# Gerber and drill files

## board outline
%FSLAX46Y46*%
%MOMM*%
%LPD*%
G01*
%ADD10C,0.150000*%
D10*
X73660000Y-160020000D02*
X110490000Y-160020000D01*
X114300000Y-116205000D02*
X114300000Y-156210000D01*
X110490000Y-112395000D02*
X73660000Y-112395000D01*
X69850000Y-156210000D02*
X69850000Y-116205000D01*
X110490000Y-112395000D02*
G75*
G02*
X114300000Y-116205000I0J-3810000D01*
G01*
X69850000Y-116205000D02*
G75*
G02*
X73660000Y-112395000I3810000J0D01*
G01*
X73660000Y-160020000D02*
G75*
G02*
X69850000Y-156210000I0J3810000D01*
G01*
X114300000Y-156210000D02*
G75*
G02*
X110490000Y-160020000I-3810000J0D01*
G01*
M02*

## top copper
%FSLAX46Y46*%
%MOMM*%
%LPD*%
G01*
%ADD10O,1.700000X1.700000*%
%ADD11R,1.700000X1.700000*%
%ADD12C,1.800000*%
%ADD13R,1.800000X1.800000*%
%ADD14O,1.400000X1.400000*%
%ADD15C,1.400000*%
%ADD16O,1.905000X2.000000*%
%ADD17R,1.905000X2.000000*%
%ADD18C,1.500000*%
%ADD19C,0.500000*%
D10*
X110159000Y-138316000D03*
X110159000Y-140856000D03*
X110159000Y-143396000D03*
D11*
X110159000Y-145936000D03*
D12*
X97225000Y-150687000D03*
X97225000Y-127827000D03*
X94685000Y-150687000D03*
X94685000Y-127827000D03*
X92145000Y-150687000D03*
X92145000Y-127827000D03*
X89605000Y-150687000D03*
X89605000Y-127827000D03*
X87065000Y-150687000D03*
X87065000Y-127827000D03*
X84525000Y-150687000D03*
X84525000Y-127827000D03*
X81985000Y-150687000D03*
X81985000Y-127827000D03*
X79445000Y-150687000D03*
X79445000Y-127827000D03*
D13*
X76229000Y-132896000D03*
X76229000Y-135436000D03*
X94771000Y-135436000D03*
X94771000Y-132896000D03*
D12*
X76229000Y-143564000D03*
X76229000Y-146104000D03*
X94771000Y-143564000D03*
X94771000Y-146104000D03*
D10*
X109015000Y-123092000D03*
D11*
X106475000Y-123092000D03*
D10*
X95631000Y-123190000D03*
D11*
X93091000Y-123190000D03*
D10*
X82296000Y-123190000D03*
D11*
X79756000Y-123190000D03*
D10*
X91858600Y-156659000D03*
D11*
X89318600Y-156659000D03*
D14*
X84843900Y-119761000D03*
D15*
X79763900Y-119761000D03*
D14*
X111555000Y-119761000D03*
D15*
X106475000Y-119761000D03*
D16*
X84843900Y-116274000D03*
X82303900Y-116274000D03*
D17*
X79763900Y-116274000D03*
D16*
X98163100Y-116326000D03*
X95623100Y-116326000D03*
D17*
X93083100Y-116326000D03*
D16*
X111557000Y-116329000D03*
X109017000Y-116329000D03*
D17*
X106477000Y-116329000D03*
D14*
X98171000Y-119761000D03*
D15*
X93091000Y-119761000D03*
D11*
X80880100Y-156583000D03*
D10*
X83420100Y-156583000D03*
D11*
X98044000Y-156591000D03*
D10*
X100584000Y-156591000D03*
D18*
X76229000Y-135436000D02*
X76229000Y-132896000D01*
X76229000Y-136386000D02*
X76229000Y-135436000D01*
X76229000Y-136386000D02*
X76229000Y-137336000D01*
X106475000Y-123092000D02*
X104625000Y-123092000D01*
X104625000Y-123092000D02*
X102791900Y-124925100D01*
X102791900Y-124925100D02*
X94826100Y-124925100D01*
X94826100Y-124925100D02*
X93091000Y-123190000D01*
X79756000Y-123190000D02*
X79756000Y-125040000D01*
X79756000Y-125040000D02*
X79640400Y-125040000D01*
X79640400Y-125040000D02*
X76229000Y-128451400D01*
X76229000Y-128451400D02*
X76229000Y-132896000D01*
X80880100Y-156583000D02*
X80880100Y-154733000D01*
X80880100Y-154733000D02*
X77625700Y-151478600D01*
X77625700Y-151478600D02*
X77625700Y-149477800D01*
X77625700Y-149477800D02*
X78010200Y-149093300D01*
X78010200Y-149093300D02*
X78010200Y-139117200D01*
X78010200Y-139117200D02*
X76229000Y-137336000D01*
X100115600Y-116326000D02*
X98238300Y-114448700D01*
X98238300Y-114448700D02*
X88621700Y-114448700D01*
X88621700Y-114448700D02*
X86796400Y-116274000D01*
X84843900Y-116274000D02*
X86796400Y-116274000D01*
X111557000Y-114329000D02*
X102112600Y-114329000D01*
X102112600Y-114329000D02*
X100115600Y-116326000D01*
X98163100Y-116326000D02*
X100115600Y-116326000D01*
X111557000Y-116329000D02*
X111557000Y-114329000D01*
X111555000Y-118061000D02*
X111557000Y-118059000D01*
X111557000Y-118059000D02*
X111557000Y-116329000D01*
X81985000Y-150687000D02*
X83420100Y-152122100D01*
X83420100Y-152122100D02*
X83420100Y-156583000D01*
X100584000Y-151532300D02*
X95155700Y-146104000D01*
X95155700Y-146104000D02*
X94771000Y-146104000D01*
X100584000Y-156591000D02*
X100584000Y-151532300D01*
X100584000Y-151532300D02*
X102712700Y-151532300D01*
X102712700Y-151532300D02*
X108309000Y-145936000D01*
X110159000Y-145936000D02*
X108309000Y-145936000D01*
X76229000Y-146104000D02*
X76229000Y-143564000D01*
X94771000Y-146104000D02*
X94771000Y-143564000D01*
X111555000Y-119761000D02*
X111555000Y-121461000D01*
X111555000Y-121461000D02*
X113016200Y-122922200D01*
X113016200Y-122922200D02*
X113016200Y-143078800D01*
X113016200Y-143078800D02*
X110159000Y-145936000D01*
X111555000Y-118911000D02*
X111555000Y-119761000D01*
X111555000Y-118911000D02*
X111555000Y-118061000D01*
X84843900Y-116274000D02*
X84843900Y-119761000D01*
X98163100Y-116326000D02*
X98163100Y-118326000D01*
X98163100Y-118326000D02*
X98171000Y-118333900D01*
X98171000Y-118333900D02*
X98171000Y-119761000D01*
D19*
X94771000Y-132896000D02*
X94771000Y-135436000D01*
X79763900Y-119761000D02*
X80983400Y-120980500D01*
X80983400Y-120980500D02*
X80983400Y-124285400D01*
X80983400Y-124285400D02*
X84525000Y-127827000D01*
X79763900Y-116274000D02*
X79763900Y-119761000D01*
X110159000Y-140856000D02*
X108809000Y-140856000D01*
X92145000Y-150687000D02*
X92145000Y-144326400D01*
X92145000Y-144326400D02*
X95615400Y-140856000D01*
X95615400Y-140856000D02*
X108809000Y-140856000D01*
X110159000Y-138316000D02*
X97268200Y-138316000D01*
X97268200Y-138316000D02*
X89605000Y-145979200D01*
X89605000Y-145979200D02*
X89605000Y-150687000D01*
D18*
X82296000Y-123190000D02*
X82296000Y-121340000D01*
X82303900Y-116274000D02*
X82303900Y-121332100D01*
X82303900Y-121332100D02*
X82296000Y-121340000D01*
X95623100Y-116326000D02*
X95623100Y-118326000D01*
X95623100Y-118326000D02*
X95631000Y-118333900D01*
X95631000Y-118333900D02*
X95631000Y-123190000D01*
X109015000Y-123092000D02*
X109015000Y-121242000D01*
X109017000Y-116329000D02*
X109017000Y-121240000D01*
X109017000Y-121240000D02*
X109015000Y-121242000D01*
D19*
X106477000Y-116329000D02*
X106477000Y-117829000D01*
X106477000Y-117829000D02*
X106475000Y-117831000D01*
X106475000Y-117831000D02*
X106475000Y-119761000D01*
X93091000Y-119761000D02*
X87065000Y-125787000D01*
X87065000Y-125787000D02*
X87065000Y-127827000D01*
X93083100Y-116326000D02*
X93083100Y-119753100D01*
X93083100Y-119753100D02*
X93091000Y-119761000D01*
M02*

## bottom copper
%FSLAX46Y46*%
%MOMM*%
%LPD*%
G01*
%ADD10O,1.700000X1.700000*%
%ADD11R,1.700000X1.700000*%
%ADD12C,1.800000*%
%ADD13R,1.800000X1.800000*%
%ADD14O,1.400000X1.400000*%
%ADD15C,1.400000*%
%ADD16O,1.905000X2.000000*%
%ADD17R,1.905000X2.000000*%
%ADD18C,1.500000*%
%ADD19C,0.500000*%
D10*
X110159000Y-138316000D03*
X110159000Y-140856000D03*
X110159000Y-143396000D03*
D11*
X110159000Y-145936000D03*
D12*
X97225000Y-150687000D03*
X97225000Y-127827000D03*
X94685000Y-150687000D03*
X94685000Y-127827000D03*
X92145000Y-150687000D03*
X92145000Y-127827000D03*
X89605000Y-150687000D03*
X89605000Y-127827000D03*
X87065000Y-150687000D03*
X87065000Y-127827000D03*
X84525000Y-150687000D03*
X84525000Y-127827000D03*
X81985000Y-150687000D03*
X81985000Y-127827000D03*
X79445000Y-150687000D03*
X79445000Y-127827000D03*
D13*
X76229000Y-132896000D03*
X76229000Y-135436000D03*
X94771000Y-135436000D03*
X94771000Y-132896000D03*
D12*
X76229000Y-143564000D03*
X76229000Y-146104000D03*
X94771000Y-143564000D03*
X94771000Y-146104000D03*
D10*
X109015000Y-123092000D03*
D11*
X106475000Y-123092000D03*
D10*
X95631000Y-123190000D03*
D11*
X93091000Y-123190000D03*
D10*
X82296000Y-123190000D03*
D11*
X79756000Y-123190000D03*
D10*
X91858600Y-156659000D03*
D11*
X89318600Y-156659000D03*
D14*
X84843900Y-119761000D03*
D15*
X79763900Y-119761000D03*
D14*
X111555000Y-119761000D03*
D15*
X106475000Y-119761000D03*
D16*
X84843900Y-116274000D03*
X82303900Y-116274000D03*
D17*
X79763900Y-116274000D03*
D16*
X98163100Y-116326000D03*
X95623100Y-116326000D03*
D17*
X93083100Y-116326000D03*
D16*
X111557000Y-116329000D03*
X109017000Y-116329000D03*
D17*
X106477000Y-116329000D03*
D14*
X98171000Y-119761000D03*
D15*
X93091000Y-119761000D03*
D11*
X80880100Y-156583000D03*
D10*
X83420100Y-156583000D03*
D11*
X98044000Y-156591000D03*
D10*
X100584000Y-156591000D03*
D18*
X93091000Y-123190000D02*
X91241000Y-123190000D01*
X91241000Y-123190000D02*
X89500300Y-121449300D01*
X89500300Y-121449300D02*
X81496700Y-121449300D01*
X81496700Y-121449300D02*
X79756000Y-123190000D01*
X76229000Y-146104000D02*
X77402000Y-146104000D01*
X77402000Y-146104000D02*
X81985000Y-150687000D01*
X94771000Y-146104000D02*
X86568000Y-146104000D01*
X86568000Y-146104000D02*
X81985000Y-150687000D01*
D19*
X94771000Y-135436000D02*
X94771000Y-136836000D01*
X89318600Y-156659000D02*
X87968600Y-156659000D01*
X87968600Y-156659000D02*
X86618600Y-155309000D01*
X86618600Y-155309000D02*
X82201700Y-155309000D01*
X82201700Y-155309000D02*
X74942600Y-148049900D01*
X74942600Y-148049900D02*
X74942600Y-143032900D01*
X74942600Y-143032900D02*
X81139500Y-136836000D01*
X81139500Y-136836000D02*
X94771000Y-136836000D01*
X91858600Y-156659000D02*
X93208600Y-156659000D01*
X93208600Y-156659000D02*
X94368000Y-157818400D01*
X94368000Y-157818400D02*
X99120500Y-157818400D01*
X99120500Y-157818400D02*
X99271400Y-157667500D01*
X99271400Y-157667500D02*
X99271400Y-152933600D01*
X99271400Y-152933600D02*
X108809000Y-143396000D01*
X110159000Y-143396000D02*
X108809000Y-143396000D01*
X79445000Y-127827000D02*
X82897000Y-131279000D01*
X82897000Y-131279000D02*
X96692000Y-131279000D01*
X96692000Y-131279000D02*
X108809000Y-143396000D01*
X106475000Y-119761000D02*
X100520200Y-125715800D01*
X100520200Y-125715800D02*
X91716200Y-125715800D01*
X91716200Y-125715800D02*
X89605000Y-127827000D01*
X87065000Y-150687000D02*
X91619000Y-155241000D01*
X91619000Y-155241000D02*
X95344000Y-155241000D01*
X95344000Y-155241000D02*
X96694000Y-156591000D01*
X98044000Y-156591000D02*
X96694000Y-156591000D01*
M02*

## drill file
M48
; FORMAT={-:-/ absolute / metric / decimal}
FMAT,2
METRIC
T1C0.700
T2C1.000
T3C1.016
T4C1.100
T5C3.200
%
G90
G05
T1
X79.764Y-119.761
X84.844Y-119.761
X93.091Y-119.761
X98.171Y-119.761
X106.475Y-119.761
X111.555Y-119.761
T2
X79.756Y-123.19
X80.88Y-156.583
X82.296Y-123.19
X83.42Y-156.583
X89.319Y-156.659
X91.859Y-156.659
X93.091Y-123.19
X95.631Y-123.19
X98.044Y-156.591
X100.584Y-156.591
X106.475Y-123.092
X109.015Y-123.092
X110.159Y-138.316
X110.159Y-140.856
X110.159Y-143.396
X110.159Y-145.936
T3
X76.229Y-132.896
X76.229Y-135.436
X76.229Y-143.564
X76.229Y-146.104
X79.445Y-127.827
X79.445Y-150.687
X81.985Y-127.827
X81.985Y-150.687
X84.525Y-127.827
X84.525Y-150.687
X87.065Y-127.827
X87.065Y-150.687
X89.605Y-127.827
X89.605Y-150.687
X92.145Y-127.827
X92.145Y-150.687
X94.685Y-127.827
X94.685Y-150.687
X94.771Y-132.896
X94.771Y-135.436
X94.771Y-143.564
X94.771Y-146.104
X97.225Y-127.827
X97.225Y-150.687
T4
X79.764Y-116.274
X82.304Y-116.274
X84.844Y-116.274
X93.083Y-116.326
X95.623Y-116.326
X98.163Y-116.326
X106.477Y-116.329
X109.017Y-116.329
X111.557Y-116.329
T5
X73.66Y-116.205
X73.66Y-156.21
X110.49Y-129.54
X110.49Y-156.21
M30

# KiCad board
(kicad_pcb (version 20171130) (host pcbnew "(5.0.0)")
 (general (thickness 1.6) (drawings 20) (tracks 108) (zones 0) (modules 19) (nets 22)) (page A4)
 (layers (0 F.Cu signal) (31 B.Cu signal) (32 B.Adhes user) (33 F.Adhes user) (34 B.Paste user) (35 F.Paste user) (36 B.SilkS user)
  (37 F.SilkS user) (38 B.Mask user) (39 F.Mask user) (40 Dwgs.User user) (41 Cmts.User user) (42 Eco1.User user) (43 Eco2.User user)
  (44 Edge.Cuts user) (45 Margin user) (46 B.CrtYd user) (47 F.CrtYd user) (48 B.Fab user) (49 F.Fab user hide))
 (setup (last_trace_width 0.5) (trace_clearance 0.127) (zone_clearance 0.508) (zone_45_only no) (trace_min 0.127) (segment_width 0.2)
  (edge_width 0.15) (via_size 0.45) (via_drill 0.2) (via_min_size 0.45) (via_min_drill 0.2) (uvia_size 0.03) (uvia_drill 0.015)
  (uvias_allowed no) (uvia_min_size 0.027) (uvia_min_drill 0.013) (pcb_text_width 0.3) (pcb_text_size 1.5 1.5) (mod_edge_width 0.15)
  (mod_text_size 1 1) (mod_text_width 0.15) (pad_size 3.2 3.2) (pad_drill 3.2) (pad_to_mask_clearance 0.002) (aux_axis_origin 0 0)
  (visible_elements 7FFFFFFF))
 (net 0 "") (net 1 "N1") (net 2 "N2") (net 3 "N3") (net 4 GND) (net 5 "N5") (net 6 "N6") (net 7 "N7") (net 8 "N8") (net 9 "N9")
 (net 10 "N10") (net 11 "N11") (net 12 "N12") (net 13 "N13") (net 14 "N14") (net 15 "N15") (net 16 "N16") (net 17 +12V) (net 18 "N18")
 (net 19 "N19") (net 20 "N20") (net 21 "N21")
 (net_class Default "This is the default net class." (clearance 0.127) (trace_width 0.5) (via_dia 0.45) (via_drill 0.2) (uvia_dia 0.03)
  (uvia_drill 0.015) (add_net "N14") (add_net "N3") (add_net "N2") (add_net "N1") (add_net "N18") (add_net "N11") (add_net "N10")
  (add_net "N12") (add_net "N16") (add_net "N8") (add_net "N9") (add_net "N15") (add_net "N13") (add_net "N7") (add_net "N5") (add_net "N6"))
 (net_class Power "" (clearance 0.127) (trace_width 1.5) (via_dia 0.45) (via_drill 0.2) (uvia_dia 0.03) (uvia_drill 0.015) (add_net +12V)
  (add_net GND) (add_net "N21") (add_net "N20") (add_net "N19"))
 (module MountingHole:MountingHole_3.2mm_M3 (layer F.Cu) (at 73.66 156.21)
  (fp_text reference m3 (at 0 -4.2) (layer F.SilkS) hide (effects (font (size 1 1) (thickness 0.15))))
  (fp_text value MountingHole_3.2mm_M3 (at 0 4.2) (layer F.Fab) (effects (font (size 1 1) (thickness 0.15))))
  (pad 1 np_thru_hole circle (at 0 0) (size 3.2 3.2) (drill 3.2) (layers *.Cu *.Mask)))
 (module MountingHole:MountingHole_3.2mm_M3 (layer F.Cu) (at 110.49 129.54)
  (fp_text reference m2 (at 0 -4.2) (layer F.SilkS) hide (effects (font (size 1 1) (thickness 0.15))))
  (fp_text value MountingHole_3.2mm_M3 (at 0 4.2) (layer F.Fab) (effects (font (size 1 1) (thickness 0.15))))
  (pad 1 np_thru_hole circle (at 0 0) (size 3.2 3.2) (drill 3.2) (layers *.Cu *.Mask)))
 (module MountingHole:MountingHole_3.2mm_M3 (layer F.Cu) (at 73.66 116.205)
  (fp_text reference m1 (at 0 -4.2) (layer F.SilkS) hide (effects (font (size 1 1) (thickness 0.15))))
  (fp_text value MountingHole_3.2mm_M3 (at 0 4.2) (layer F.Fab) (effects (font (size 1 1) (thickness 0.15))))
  (pad "" np_thru_hole circle (at 0 0) (size 3.2 3.2) (drill 3.2) (layers *.Cu *.Mask)))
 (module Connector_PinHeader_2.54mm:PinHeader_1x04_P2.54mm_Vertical (layer F.Cu) (at 110.159 145.936 180)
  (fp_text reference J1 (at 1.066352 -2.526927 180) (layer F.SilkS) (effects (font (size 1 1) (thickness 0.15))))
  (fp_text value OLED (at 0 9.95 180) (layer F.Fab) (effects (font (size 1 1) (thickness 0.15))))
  (pad 4 thru_hole oval (at 0 7.62 180) (size 1.7 1.7) (drill 1) (layers *.Cu *.Mask) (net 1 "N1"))
  (pad 3 thru_hole oval (at 0 5.08 180) (size 1.7 1.7) (drill 1) (layers *.Cu *.Mask) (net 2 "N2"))
  (pad 2 thru_hole oval (at 0 2.54 180) (size 1.7 1.7) (drill 1) (layers *.Cu *.Mask) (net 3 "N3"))
  (pad 1 thru_hole rect (at 0 0 180) (size 1.7 1.7) (drill 1) (layers *.Cu *.Mask) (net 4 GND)))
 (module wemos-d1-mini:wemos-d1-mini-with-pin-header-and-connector (layer F.Cu) (at 88.335 139.257)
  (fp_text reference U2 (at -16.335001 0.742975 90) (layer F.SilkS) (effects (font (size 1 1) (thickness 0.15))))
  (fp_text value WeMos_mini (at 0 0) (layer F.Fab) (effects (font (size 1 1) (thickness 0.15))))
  (pad 8 thru_hole circle (at 8.89 11.43) (size 1.8 1.8) (drill 1.016) (layers *.Cu *.Mask) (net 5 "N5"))
  (pad 9 thru_hole circle (at 8.89 -11.43) (size 1.8 1.8) (drill 1.016) (layers *.Cu *.Mask) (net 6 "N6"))
  (pad 7 thru_hole circle (at 6.35 11.43) (size 1.8 1.8) (drill 1.016) (layers *.Cu *.Mask) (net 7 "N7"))
  (pad 10 thru_hole circle (at 6.35 -11.43) (size 1.8 1.8) (drill 1.016) (layers *.Cu *.Mask) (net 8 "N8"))
  (pad 6 thru_hole circle (at 3.81 11.43) (size 1.8 1.8) (drill 1.016) (layers *.Cu *.Mask) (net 2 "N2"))
  (pad 11 thru_hole circle (at 3.81 -11.43) (size 1.8 1.8) (drill 1.016) (layers *.Cu *.Mask) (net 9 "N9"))
  (pad 5 thru_hole circle (at 1.27 11.43) (size 1.8 1.8) (drill 1.016) (layers *.Cu *.Mask) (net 1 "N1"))
  (pad 12 thru_hole circle (at 1.27 -11.43) (size 1.8 1.8) (drill 1.016) (layers *.Cu *.Mask) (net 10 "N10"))
  (pad 4 thru_hole circle (at -1.27 11.43) (size 1.8 1.8) (drill 1.016) (layers *.Cu *.Mask) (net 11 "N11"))
  (pad 13 thru_hole circle (at -1.27 -11.43) (size 1.8 1.8) (drill 1.016) (layers *.Cu *.Mask) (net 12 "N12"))
  (pad 3 thru_hole circle (at -3.81 11.43) (size 1.8 1.8) (drill 1.016) (layers *.Cu *.Mask) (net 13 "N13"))
  (pad 14 thru_hole circle (at -3.81 -11.43) (size 1.8 1.8) (drill 1.016) (layers *.Cu *.Mask) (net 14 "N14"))
  (pad 2 thru_hole circle (at -6.35 11.43) (size 1.8 1.8) (drill 1.016) (layers *.Cu *.Mask) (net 4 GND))
  (pad 15 thru_hole circle (at -6.35 -11.43) (size 1.8 1.8) (drill 1.016) (layers *.Cu *.Mask) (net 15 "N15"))
  (pad 1 thru_hole circle (at -8.89 11.43) (size 1.8 1.8) (drill 1.016) (layers *.Cu *.Mask) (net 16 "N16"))
  (pad 16 thru_hole circle (at -8.89 -11.43) (size 1.8 1.8) (drill 1.016) (layers *.Cu *.Mask) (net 3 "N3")))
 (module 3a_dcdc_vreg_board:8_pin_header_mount (layer B.Cu) (at 85.5 139.5)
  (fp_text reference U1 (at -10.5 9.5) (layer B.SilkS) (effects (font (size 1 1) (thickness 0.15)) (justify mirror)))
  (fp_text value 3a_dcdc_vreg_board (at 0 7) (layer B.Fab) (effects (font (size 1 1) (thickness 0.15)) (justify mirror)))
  (pad 7 thru_hole rect (at -9.271 -6.604) (size 1.8 1.8) (drill 1.016) (layers *.Cu *.Mask) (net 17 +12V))
  (pad 5 thru_hole rect (at -9.271 -4.064) (size 1.8 1.8) (drill 1.016) (layers *.Cu *.Mask) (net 17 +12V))
  (pad 6 thru_hole rect (at 9.271 -4.064) (size 1.8 1.8) (drill 1.016) (layers *.Cu *.Mask) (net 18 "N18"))
  (pad 8 thru_hole rect (at 9.271 -6.604 270) (size 1.8 1.8) (drill 1.016) (layers *.Cu *.Mask) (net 18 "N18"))
  (pad 3 thru_hole circle (at -9.271 4.064) (size 1.8 1.8) (drill 1.016) (layers *.Cu *.Mask) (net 4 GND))
  (pad 1 thru_hole circle (at -9.271 6.604) (size 1.8 1.8) (drill 1.016) (layers *.Cu *.Mask) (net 4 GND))
  (pad 4 thru_hole circle (at 9.271 4.064) (size 1.8 1.8) (drill 1.016) (layers *.Cu *.Mask) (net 4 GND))
  (pad 2 thru_hole circle (at 9.271 6.604) (size 1.8 1.8) (drill 1.016) (layers *.Cu *.Mask) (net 4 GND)))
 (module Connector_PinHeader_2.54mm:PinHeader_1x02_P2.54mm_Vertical (layer F.Cu) (at 106.475 123.092 90)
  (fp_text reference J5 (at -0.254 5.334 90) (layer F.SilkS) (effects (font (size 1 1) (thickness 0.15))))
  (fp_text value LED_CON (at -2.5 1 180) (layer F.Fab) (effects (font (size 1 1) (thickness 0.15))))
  (pad 2 thru_hole oval (at 0 2.54 90) (size 1.7 1.7) (drill 1) (layers *.Cu *.Mask) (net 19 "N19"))
  (pad 1 thru_hole rect (at 0 0 90) (size 1.7 1.7) (drill 1) (layers *.Cu *.Mask) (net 17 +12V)))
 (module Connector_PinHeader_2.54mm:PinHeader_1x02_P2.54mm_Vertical (layer F.Cu) (at 93.091 123.19 90)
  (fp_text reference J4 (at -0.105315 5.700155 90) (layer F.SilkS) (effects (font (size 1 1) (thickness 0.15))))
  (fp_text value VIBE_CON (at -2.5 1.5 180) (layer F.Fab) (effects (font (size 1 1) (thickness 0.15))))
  (pad 2 thru_hole oval (at 0 2.54 90) (size 1.7 1.7) (drill 1) (layers *.Cu *.Mask) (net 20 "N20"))
  (pad 1 thru_hole rect (at 0 0 90) (size 1.7 1.7) (drill 1) (layers *.Cu *.Mask) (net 17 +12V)))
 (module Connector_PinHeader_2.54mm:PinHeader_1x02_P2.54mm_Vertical (layer F.Cu) (at 79.756 123.19 90)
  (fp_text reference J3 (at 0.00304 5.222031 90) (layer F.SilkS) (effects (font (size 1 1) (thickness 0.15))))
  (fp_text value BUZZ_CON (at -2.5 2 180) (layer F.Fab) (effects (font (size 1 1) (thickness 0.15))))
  (pad 2 thru_hole oval (at 0 2.54 90) (size 1.7 1.7) (drill 1) (layers *.Cu *.Mask) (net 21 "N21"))
  (pad 1 thru_hole rect (at 0 0 90) (size 1.7 1.7) (drill 1) (layers *.Cu *.Mask) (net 17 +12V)))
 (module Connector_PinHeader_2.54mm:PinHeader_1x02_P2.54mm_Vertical (layer F.Cu) (at 89.3186 156.659 90)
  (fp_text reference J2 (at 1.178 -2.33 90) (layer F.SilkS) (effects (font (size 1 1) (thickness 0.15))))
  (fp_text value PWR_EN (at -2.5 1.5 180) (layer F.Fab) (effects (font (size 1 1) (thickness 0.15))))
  (pad 2 thru_hole oval (at 0 2.54 90) (size 1.7 1.7) (drill 1) (layers *.Cu *.Mask) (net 3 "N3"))
  (pad 1 thru_hole rect (at 0 0 90) (size 1.7 1.7) (drill 1) (layers *.Cu *.Mask) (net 18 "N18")))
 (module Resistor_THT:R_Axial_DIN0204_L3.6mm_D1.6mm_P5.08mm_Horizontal (layer F.Cu) (at 79.7639 119.761)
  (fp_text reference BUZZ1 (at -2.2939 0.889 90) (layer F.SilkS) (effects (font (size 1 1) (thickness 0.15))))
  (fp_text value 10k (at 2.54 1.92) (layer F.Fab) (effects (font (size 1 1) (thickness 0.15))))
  (pad 2 thru_hole oval (at 5.08 0) (size 1.4 1.4) (drill 0.7) (layers *.Cu *.Mask) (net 4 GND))
  (pad 1 thru_hole circle (at 0 0) (size 1.4 1.4) (drill 0.7) (layers *.Cu *.Mask) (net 14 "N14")))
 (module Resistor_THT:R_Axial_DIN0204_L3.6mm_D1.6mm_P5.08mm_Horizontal (layer F.Cu) (at 106.475 119.761)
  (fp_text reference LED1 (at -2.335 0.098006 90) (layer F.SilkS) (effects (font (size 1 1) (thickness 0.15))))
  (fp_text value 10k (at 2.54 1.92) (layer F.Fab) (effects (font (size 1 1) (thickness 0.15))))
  (pad 2 thru_hole oval (at 5.08 0) (size 1.4 1.4) (drill 0.7) (layers *.Cu *.Mask) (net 4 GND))
  (pad 1 thru_hole circle (at 0 0) (size 1.4 1.4) (drill 0.7) (layers *.Cu *.Mask) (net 10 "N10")))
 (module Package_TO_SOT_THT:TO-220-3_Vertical (layer F.Cu) (at 79.7639 116.274)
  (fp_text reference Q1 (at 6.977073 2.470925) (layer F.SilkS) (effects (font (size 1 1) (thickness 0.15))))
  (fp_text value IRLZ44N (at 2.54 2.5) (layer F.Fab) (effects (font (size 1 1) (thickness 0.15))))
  (pad 3 thru_hole oval (at 5.08 0) (size 1.905 2) (drill 1.1) (layers *.Cu *.Mask) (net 4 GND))
  (pad 2 thru_hole oval (at 2.54 0) (size 1.905 2) (drill 1.1) (layers *.Cu *.Mask) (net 21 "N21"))
  (pad 1 thru_hole rect (at 0 0) (size 1.905 2) (drill 1.1) (layers *.Cu *.Mask) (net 14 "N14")))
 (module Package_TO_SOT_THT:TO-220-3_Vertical (layer F.Cu) (at 93.0831 116.326)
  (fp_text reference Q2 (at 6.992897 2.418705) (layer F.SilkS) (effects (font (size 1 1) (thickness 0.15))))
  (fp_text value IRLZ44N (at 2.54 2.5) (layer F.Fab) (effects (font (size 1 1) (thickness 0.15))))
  (pad 3 thru_hole oval (at 5.08 0) (size 1.905 2) (drill 1.1) (layers *.Cu *.Mask) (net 4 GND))
  (pad 2 thru_hole oval (at 2.54 0) (size 1.905 2) (drill 1.1) (layers *.Cu *.Mask) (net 20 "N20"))
  (pad 1 thru_hole rect (at 0 0) (size 1.905 2) (drill 1.1) (layers *.Cu *.Mask) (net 12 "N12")))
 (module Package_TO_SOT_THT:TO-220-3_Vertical (layer F.Cu) (at 106.477 116.329)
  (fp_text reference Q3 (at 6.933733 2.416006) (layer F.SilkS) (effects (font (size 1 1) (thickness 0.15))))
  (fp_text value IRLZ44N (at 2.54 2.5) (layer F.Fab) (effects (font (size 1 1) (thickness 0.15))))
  (pad 3 thru_hole oval (at 5.08 0) (size 1.905 2) (drill 1.1) (layers *.Cu *.Mask) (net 4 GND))
  (pad 2 thru_hole oval (at 2.54 0) (size 1.905 2) (drill 1.1) (layers *.Cu *.Mask) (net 19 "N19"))
  (pad 1 thru_hole rect (at 0 0) (size 1.905 2) (drill 1.1) (layers *.Cu *.Mask) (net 10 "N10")))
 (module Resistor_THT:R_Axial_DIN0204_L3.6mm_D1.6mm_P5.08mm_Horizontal (layer F.Cu) (at 93.091 119.761)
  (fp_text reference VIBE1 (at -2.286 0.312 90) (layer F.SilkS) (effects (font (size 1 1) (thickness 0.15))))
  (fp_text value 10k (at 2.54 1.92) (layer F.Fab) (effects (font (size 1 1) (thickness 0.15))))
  (pad 2 thru_hole oval (at 5.08 0) (size 1.4 1.4) (drill 0.7) (layers *.Cu *.Mask) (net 4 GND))
  (pad 1 thru_hole circle (at 0 0) (size 1.4 1.4) (drill 0.7) (layers *.Cu *.Mask) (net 12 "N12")))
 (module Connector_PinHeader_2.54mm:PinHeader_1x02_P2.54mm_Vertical (layer F.Cu) (at 80.8801 156.583 90)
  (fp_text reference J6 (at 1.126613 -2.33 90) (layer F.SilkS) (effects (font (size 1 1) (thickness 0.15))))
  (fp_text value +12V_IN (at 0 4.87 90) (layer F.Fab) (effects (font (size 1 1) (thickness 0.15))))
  (pad 1 thru_hole rect (at 0 0 90) (size 1.7 1.7) (drill 1) (layers *.Cu *.Mask) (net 17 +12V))
  (pad 2 thru_hole oval (at 0 2.54 90) (size 1.7 1.7) (drill 1) (layers *.Cu *.Mask) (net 4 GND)))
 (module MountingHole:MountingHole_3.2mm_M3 (layer F.Cu) (at 110.49 156.21)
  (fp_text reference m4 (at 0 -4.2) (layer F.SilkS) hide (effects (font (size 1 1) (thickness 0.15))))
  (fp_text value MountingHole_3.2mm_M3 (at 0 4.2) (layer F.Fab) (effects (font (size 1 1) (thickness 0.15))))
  (pad 1 np_thru_hole circle (at 0 0) (size 3.2 3.2) (drill 3.2) (layers *.Cu *.Mask)))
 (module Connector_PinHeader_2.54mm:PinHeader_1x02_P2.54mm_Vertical (layer F.Cu) (at 98.044 156.591 90)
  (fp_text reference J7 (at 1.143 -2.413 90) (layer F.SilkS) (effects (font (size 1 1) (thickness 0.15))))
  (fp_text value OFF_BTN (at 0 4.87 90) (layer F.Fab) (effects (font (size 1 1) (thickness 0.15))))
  (pad 1 thru_hole rect (at 0 0 90) (size 1.7 1.7) (drill 1) (layers *.Cu *.Mask) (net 11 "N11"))
  (pad 2 thru_hole oval (at 0 2.54 90) (size 1.7 1.7) (drill 1) (layers *.Cu *.Mask) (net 4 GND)))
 (gr_line (start 73.66 160.02) (end 110.49 160.02) (layer Edge.Cuts) (width 0.15))
 (gr_line (start 114.3 116.205) (end 114.3 156.21) (layer Edge.Cuts) (width 0.15))
 (gr_line (start 110.49 112.395) (end 73.66 112.395) (layer Edge.Cuts) (width 0.15))
 (gr_line (start 69.85 156.21) (end 69.85 116.205) (layer Edge.Cuts) (width 0.15))
 (gr_arc (start 110.49 116.205) (end 114.3 116.205) (angle -90) (layer Edge.Cuts) (width 0.15))
 (gr_arc (start 73.66 116.205) (end 73.66 112.395) (angle -90) (layer Edge.Cuts) (width 0.15))
 (gr_arc (start 73.66 156.21) (end 69.85 156.21) (angle -90) (layer Edge.Cuts) (width 0.15))
 (gr_arc (start 110.49 156.21) (end 110.49 160.02) (angle -90) (layer Edge.Cuts) (width 0.15))
 (segment (start 76.229 135.436) (end 76.229 132.896) (width 1.5) (layer F.Cu) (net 17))
 (segment (start 76.229 136.386) (end 76.229 135.436) (width 1.5) (layer F.Cu) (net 17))
 (segment (start 76.229 136.386) (end 76.229 137.336) (width 1.5) (layer F.Cu) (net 17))
 (segment (start 106.475 123.092) (end 104.625 123.092) (width 1.5) (layer F.Cu) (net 17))
 (segment (start 104.625 123.092) (end 102.7919 124.9251) (width 1.5) (layer F.Cu) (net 17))
 (segment (start 102.7919 124.9251) (end 94.8261 124.9251) (width 1.5) (layer F.Cu) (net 17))
 (segment (start 94.8261 124.9251) (end 93.091 123.19) (width 1.5) (layer F.Cu) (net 17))
 (segment (start 93.091 123.19) (end 91.241 123.19) (width 1.5) (layer B.Cu) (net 17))
 (segment (start 91.241 123.19) (end 89.5003 121.4493) (width 1.5) (layer B.Cu) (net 17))
 (segment (start 89.5003 121.4493) (end 81.4967 121.4493) (width 1.5) (layer B.Cu) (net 17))
 (segment (start 81.4967 121.4493) (end 79.756 123.19) (width 1.5) (layer B.Cu) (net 17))
 (segment (start 79.756 123.19) (end 79.756 125.04) (width 1.5) (layer F.Cu) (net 17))
 (segment (start 79.756 125.04) (end 79.6404 125.04) (width 1.5) (layer F.Cu) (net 17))
 (segment (start 79.6404 125.04) (end 76.229 128.4514) (width 1.5) (layer F.Cu) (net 17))
 (segment (start 76.229 128.4514) (end 76.229 132.896) (width 1.5) (layer F.Cu) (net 17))
 (segment (start 80.8801 156.583) (end 80.8801 154.733) (width 1.5) (layer F.Cu) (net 17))
 (segment (start 80.8801 154.733) (end 77.6257 151.4786) (width 1.5) (layer F.Cu) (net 17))
 (segment (start 77.6257 151.4786) (end 77.6257 149.4778) (width 1.5) (layer F.Cu) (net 17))
 (segment (start 77.6257 149.4778) (end 78.0102 149.0933) (width 1.5) (layer F.Cu) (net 17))
 (segment (start 78.0102 149.0933) (end 78.0102 139.1172) (width 1.5) (layer F.Cu) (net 17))
 (segment (start 78.0102 139.1172) (end 76.229 137.336) (width 1.5) (layer F.Cu) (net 17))
 (segment (start 100.1156 116.326) (end 98.2383 114.4487) (width 1.5) (layer F.Cu) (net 4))
 (segment (start 98.2383 114.4487) (end 88.6217 114.4487) (width 1.5) (layer F.Cu) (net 4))
 (segment (start 88.6217 114.4487) (end 86.7964 116.274) (width 1.5) (layer F.Cu) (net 4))
 (segment (start 84.8439 116.274) (end 86.7964 116.274) (width 1.5) (layer F.Cu) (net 4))
 (segment (start 111.557 114.329) (end 102.1126 114.329) (width 1.5) (layer F.Cu) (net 4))
 (segment (start 102.1126 114.329) (end 100.1156 116.326) (width 1.5) (layer F.Cu) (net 4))
 (segment (start 98.1631 116.326) (end 100.1156 116.326) (width 1.5) (layer F.Cu) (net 4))
 (segment (start 111.557 116.329) (end 111.557 114.329) (width 1.5) (layer F.Cu) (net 4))
 (segment (start 111.555 118.061) (end 111.557 118.059) (width 1.5) (layer F.Cu) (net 4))
 (segment (start 111.557 118.059) (end 111.557 116.329) (width 1.5) (layer F.Cu) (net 4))
 (segment (start 81.985 150.687) (end 83.4201 152.1221) (width 1.5) (layer F.Cu) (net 4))
 (segment (start 83.4201 152.1221) (end 83.4201 156.583) (width 1.5) (layer F.Cu) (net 4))
 (segment (start 100.584 151.5323) (end 95.1557 146.104) (width 1.5) (layer F.Cu) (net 4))
 (segment (start 95.1557 146.104) (end 94.771 146.104) (width 1.5) (layer F.Cu) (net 4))
 (segment (start 100.584 156.591) (end 100.584 151.5323) (width 1.5) (layer F.Cu) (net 4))
 (segment (start 100.584 151.5323) (end 102.7127 151.5323) (width 1.5) (layer F.Cu) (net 4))
 (segment (start 102.7127 151.5323) (end 108.309 145.936) (width 1.5) (layer F.Cu) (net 4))
 (segment (start 110.159 145.936) (end 108.309 145.936) (width 1.5) (layer F.Cu) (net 4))
 (segment (start 76.229 146.104) (end 77.402 146.104) (width 1.5) (layer B.Cu) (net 4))
 (segment (start 77.402 146.104) (end 81.985 150.687) (width 1.5) (layer B.Cu) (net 4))
 (segment (start 94.771 146.104) (end 86.568 146.104) (width 1.5) (layer B.Cu) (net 4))
 (segment (start 86.568 146.104) (end 81.985 150.687) (width 1.5) (layer B.Cu) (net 4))
 (segment (start 76.229 146.104) (end 76.229 143.564) (width 1.5) (layer F.Cu) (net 4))
 (segment (start 94.771 146.104) (end 94.771 143.564) (width 1.5) (layer F.Cu) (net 4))
 (segment (start 111.555 119.761) (end 111.555 121.461) (width 1.5) (layer F.Cu) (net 4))
 (segment (start 111.555 121.461) (end 113.0162 122.9222) (width 1.5) (layer F.Cu) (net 4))
 (segment (start 113.0162 122.9222) (end 113.0162 143.0788) (width 1.5) (layer F.Cu) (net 4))
 (segment (start 113.0162 143.0788) (end 110.159 145.936) (width 1.5) (layer F.Cu) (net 4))
 (segment (start 111.555 118.911) (end 111.555 119.761) (width 1.5) (layer F.Cu) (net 4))
 (segment (start 111.555 118.911) (end 111.555 118.061) (width 1.5) (layer F.Cu) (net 4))
 (segment (start 84.8439 116.274) (end 84.8439 119.761) (width 1.5) (layer F.Cu) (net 4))
 (segment (start 98.1631 116.326) (end 98.1631 118.326) (width 1.5) (layer F.Cu) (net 4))
 (segment (start 98.1631 118.326) (end 98.171 118.3339) (width 1.5) (layer F.Cu) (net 4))
 (segment (start 98.171 118.3339) (end 98.171 119.761) (width 1.5) (layer F.Cu) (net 4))
 (segment (start 94.771 135.436) (end 94.771 136.836) (width 0.5) (layer B.Cu) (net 18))
 (segment (start 89.3186 156.659) (end 87.9686 156.659) (width 0.5) (layer B.Cu) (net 18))
 (segment (start 87.9686 156.659) (end 86.6186 155.309) (width 0.5) (layer B.Cu) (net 18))
 (segment (start 86.6186 155.309) (end 82.2017 155.309) (width 0.5) (layer B.Cu) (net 18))
 (segment (start 82.2017 155.309) (end 74.9426 148.0499) (width 0.5) (layer B.Cu) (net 18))
 (segment (start 74.9426 148.0499) (end 74.9426 143.0329) (width 0.5) (layer B.Cu) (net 18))
 (segment (start 74.9426 143.0329) (end 81.1395 136.836) (width 0.5) (layer B.Cu) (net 18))
 (segment (start 81.1395 136.836) (end 94.771 136.836) (width 0.5) (layer B.Cu) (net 18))
 (segment (start 94.771 132.896) (end 94.771 135.436) (width 0.5) (layer F.Cu) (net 18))
 (segment (start 79.7639 119.761) (end 80.9834 120.9805) (width 0.5) (layer F.Cu) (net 14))
 (segment (start 80.9834 120.9805) (end 80.9834 124.2854) (width 0.5) (layer F.Cu) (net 14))
 (segment (start 80.9834 124.2854) (end 84.525 127.827) (width 0.5) (layer F.Cu) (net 14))
 (segment (start 79.7639 116.274) (end 79.7639 119.761) (width 0.5) (layer F.Cu) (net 14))
 (segment (start 91.8586 156.659) (end 93.2086 156.659) (width 0.5) (layer B.Cu) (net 3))
 (segment (start 93.2086 156.659) (end 94.368 157.8184) (width 0.5) (layer B.Cu) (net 3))
 (segment (start 94.368 157.8184) (end 99.1205 157.8184) (width 0.5) (layer B.Cu) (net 3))
 (segment (start 99.1205 157.8184) (end 99.2714 157.6675) (width 0.5) (layer B.Cu) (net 3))
 (segment (start 99.2714 157.6675) (end 99.2714 152.9336) (width 0.5) (layer B.Cu) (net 3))
 (segment (start 99.2714 152.9336) (end 108.809 143.396) (width 0.5) (layer B.Cu) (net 3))
 (segment (start 110.159 143.396) (end 108.809 143.396) (width 0.5) (layer B.Cu) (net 3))
 (segment (start 79.445 127.827) (end 82.897 131.279) (width 0.5) (layer B.Cu) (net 3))
 (segment (start 82.897 131.279) (end 96.692 131.279) (width 0.5) (layer B.Cu) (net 3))
 (segment (start 96.692 131.279) (end 108.809 143.396) (width 0.5) (layer B.Cu) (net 3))
 (segment (start 110.159 140.856) (end 108.809 140.856) (width 0.5) (layer F.Cu) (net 2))
 (segment (start 92.145 150.687) (end 92.145 144.3264) (width 0.5) (layer F.Cu) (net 2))
 (segment (start 92.145 144.3264) (end 95.6154 140.856) (width 0.5) (layer F.Cu) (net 2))
 (segment (start 95.6154 140.856) (end 108.809 140.856) (width 0.5) (layer F.Cu) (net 2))
 (segment (start 110.159 138.316) (end 97.2682 138.316) (width 0.5) (layer F.Cu) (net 1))
 (segment (start 97.2682 138.316) (end 89.605 145.9792) (width 0.5) (layer F.Cu) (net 1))
 (segment (start 89.605 145.9792) (end 89.605 150.687) (width 0.5) (layer F.Cu) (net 1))
 (segment (start 82.296 123.19) (end 82.296 121.34) (width 1.5) (layer F.Cu) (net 21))
 (segment (start 82.3039 116.274) (end 82.3039 121.3321) (width 1.5) (layer F.Cu) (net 21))
 (segment (start 82.3039 121.3321) (end 82.296 121.34) (width 1.5) (layer F.Cu) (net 21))
 (segment (start 95.6231 116.326) (end 95.6231 118.326) (width 1.5) (layer F.Cu) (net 20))
 (segment (start 95.6231 118.326) (end 95.631 118.3339) (width 1.5) (layer F.Cu) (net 20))
 (segment (start 95.631 118.3339) (end 95.631 123.19) (width 1.5) (layer F.Cu) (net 20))
 (segment (start 109.015 123.092) (end 109.015 121.242) (width 1.5) (layer F.Cu) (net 19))
 (segment (start 109.017 116.329) (end 109.017 121.24) (width 1.5) (layer F.Cu) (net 19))
 (segment (start 109.017 121.24) (end 109.015 121.242) (width 1.5) (layer F.Cu) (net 19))
 (segment (start 106.475 119.761) (end 100.5202 125.7158) (width 0.5) (layer B.Cu) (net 10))
 (segment (start 100.5202 125.7158) (end 91.7162 125.7158) (width 0.5) (layer B.Cu) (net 10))
 (segment (start 91.7162 125.7158) (end 89.605 127.827) (width 0.5) (layer B.Cu) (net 10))
 (segment (start 106.477 116.329) (end 106.477 117.829) (width 0.5) (layer F.Cu) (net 10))
 (segment (start 106.477 117.829) (end 106.475 117.831) (width 0.5) (layer F.Cu) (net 10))
 (segment (start 106.475 117.831) (end 106.475 119.761) (width 0.5) (layer F.Cu) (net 10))
 (segment (start 93.091 119.761) (end 87.065 125.787) (width 0.5) (layer F.Cu) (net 12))
 (segment (start 87.065 125.787) (end 87.065 127.827) (width 0.5) (layer F.Cu) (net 12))
 (segment (start 93.0831 116.326) (end 93.0831 119.7531) (width 0.5) (layer F.Cu) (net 12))
 (segment (start 93.0831 119.7531) (end 93.091 119.761) (width 0.5) (layer F.Cu) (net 12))
 (segment (start 87.065 150.687) (end 91.619 155.241) (width 0.5) (layer B.Cu) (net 11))
 (segment (start 91.619 155.241) (end 95.344 155.241) (width 0.5) (layer B.Cu) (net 11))
 (segment (start 95.344 155.241) (end 96.694 156.591) (width 0.5) (layer B.Cu) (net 11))
 (segment (start 98.044 156.591) (end 96.694 156.591) (width 0.5) (layer B.Cu) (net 11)))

